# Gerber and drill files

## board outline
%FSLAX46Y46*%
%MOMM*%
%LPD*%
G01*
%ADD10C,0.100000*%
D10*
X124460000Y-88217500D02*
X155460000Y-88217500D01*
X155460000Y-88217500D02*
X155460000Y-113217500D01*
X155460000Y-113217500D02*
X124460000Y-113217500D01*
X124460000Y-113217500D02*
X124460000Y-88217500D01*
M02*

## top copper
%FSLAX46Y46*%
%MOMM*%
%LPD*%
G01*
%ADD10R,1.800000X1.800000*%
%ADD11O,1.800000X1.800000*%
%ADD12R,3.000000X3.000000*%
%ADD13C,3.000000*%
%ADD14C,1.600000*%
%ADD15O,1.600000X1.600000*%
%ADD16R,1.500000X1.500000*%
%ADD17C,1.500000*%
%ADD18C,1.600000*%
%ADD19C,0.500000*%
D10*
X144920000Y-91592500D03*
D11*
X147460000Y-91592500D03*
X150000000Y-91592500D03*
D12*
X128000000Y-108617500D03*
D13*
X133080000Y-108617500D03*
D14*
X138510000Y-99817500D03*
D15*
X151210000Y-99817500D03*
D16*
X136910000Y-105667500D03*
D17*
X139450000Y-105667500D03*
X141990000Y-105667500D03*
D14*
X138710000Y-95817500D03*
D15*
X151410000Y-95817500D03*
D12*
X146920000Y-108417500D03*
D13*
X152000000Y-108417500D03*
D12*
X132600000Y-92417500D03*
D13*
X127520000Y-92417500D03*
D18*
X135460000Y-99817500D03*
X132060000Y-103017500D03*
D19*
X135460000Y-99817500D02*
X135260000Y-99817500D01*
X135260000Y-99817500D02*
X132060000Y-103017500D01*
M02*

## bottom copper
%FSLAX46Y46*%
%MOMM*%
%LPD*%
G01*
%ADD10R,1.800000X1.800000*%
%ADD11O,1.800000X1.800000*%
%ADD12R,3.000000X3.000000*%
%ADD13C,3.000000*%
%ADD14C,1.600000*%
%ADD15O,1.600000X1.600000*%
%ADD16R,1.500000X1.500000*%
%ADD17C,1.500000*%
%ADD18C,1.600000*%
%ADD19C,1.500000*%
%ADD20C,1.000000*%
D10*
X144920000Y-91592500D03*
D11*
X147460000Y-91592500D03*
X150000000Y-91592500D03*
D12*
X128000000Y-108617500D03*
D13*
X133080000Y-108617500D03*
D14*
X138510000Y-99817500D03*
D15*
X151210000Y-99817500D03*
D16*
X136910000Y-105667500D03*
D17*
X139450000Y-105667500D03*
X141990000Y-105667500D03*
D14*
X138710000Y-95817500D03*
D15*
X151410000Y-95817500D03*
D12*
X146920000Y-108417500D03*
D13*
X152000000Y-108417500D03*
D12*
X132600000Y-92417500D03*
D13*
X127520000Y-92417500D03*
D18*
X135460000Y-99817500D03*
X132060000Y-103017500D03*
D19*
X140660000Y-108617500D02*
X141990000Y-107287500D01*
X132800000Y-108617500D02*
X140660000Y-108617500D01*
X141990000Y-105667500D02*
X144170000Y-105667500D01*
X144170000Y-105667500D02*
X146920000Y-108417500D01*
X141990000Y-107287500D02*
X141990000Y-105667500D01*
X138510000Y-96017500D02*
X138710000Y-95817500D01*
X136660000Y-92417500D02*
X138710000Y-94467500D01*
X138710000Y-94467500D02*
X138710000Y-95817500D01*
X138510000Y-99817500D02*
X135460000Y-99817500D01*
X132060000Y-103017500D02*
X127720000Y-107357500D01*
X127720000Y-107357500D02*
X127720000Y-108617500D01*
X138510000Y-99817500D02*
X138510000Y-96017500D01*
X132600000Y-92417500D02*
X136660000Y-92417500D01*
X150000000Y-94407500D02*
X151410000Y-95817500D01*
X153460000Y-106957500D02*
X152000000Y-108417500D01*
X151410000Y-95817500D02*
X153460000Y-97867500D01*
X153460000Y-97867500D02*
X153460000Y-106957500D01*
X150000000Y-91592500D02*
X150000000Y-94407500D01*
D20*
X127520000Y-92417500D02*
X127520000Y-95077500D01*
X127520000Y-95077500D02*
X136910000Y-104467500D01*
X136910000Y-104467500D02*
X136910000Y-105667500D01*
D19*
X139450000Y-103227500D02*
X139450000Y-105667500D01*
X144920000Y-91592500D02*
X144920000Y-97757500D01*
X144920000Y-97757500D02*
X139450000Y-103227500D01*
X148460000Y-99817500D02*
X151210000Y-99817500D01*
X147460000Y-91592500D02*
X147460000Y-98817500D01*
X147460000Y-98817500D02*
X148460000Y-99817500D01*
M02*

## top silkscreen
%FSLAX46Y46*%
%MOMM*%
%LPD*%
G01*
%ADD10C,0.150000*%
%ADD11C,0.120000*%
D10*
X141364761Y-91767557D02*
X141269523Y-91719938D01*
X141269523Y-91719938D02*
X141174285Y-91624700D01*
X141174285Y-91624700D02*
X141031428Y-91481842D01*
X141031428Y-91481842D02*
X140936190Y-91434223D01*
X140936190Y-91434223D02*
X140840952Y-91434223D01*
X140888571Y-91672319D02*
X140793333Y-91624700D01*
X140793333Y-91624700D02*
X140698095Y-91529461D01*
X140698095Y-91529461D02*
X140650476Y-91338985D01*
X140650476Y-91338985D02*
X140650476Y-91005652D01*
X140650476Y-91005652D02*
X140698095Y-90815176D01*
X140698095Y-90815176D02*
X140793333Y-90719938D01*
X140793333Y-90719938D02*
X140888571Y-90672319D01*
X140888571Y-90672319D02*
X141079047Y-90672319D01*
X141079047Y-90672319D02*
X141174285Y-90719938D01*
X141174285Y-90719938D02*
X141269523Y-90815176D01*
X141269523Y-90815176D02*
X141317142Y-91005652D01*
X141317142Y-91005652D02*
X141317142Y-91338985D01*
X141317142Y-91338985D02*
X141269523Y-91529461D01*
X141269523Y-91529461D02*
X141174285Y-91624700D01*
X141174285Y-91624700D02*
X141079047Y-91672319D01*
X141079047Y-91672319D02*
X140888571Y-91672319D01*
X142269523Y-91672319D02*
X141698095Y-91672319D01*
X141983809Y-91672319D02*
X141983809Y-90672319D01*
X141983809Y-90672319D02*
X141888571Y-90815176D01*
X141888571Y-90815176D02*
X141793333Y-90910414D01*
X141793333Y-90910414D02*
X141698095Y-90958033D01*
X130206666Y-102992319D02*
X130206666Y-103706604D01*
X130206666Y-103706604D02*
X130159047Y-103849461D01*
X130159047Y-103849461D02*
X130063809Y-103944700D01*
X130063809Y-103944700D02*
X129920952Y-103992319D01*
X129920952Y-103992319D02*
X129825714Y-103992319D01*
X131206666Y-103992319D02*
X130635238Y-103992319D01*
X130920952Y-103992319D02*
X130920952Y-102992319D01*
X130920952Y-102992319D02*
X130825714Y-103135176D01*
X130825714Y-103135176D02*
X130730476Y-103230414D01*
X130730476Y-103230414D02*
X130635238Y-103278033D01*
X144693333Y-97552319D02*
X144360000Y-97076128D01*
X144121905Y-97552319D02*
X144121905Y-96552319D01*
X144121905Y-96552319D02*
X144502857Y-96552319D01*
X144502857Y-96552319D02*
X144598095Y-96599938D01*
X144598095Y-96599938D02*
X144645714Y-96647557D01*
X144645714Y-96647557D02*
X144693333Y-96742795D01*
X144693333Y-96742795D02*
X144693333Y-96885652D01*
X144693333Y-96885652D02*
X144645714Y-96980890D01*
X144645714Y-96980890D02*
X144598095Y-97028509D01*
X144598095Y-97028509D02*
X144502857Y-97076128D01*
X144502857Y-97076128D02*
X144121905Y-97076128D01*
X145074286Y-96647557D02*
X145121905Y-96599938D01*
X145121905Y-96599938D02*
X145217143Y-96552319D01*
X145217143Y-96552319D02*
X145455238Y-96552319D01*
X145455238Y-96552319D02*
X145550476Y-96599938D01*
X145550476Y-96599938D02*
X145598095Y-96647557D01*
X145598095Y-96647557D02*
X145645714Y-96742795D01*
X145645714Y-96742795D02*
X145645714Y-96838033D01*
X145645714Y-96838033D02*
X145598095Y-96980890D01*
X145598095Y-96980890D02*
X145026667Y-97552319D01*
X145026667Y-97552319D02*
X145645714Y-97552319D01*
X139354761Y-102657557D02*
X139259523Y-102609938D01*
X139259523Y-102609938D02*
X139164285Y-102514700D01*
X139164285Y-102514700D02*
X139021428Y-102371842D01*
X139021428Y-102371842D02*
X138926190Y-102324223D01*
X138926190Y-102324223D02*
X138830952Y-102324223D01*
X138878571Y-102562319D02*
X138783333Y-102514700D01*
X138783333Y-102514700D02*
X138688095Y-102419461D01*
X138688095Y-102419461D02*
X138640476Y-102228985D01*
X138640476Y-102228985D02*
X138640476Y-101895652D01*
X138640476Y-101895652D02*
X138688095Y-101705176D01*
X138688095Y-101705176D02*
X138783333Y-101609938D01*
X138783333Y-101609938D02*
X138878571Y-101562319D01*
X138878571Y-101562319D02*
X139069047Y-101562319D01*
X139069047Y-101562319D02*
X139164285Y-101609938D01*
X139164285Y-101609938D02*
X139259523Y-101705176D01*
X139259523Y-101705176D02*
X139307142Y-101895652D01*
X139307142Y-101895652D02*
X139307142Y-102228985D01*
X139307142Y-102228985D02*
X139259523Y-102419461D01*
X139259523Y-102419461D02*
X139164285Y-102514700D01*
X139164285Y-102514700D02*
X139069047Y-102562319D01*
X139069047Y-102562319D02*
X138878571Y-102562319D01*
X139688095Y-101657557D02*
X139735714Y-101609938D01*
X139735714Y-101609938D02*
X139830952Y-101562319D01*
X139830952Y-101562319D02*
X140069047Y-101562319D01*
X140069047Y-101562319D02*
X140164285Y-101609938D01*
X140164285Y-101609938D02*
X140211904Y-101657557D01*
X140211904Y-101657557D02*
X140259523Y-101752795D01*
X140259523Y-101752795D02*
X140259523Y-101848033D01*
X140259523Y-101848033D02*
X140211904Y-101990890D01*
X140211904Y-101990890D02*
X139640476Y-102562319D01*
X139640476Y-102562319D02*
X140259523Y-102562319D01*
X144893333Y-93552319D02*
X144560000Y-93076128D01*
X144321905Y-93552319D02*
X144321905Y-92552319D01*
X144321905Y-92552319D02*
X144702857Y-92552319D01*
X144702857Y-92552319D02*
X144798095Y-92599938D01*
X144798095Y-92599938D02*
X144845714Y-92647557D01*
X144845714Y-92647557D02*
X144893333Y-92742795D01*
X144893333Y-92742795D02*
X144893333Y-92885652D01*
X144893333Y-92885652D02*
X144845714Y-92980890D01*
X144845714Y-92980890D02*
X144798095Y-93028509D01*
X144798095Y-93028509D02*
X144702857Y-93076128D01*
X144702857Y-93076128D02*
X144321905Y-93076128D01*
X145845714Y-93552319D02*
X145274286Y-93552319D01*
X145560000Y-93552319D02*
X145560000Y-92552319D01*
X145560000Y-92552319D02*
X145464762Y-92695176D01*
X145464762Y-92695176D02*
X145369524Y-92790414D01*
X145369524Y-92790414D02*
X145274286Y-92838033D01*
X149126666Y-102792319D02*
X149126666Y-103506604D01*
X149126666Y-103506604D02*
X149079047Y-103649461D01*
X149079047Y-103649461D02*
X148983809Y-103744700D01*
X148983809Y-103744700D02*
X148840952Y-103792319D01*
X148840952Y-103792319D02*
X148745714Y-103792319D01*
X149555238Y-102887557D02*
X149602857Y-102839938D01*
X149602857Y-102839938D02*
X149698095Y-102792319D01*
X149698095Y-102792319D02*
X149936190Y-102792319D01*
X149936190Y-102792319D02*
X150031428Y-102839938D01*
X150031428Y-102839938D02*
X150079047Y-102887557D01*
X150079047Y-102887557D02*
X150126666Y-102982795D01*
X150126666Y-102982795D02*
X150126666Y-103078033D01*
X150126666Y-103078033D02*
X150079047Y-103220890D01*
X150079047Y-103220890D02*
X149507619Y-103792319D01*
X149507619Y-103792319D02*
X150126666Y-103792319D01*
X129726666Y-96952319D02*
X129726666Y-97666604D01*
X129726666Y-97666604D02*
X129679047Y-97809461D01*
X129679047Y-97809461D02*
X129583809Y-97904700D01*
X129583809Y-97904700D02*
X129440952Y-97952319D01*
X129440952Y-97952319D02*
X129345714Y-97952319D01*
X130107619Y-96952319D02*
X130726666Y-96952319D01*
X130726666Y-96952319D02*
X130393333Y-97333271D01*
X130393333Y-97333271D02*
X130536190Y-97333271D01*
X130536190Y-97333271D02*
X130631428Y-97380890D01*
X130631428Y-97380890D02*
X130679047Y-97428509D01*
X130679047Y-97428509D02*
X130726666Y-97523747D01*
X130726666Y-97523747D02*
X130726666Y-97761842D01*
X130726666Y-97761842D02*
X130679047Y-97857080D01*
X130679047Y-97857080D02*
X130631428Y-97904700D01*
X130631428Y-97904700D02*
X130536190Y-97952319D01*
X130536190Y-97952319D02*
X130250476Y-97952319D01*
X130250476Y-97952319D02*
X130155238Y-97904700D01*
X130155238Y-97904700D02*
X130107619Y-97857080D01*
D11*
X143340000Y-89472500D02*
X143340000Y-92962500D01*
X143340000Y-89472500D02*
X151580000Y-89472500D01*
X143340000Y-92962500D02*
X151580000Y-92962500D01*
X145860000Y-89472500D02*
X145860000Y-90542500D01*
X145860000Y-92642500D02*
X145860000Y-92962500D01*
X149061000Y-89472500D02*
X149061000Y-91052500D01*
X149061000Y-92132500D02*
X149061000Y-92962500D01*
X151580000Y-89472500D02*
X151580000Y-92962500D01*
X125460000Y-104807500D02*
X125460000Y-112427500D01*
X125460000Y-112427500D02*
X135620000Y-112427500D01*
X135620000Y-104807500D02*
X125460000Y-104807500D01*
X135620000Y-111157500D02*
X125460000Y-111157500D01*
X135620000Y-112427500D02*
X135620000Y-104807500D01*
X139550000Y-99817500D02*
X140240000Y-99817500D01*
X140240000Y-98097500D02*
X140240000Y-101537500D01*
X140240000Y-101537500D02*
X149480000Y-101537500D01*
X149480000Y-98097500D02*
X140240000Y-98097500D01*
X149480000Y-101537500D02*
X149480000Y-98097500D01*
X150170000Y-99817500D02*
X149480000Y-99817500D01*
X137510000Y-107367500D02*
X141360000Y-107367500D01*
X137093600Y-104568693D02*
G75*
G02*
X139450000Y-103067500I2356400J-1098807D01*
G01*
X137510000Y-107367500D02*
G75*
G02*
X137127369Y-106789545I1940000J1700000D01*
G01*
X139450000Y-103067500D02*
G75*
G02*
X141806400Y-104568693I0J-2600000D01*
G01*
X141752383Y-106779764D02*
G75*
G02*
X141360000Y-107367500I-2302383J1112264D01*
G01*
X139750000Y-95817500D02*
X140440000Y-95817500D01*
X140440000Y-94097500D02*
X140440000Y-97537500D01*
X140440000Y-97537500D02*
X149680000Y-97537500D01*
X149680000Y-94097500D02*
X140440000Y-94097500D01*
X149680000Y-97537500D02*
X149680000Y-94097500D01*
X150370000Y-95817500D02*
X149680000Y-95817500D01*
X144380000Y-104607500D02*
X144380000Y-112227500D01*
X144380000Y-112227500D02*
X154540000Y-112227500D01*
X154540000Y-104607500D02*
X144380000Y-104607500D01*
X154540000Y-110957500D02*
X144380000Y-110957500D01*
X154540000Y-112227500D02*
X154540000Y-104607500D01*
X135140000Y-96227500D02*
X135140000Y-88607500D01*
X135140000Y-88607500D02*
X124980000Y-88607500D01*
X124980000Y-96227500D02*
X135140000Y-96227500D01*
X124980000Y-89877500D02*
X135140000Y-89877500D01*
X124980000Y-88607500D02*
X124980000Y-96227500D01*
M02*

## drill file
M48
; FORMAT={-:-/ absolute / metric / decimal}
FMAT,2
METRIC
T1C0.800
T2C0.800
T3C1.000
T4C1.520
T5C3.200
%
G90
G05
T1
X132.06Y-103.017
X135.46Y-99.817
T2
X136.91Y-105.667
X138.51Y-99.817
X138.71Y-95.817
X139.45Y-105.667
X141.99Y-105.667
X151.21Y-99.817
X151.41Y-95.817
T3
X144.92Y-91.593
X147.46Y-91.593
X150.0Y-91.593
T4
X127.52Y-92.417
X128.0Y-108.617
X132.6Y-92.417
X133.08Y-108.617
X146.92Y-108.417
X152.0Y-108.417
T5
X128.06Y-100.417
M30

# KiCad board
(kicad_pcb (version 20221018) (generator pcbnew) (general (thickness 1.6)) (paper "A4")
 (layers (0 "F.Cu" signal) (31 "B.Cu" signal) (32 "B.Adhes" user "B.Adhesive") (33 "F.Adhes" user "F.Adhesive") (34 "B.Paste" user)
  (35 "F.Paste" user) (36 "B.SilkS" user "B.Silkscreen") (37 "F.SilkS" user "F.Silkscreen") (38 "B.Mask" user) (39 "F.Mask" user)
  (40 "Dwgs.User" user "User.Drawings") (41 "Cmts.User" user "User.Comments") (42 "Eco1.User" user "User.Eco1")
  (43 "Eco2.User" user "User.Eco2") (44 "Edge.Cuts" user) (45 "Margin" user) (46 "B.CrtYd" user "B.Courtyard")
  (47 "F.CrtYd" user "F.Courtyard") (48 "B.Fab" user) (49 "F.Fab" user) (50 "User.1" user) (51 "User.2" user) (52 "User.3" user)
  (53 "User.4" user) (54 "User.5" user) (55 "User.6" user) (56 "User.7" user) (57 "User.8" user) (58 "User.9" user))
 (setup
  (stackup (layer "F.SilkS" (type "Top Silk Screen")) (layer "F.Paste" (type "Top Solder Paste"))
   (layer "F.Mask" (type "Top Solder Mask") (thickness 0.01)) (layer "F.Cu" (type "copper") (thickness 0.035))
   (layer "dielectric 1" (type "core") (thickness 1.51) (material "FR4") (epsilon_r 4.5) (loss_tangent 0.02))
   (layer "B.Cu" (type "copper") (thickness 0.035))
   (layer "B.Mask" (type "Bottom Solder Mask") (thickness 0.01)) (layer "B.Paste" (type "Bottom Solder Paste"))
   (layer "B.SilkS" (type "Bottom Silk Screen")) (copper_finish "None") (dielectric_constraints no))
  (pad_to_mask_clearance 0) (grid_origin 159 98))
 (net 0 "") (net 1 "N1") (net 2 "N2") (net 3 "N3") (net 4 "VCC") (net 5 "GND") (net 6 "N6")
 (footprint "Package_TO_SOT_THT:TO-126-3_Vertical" (layer "F.Cu") (at 144.92 91.5925)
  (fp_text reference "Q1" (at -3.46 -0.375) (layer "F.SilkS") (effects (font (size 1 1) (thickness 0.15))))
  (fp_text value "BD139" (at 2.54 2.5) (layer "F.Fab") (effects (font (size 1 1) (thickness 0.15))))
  (fp_line (start -1.58 -2.12) (end -1.58 1.37) (stroke (width 0.12) (type solid)) (layer "F.SilkS"))
  (fp_line (start -1.58 -2.12) (end 6.66 -2.12) (stroke (width 0.12) (type solid)) (layer "F.SilkS"))
  (fp_line (start -1.58 1.37) (end 6.66 1.37) (stroke (width 0.12) (type solid)) (layer "F.SilkS"))
  (fp_line (start 0.94 -2.12) (end 0.94 -1.05) (stroke (width 0.12) (type solid)) (layer "F.SilkS"))
  (fp_line (start 0.94 1.05) (end 0.94 1.37) (stroke (width 0.12) (type solid)) (layer "F.SilkS"))
  (fp_line (start 4.141 -2.12) (end 4.141 -0.54) (stroke (width 0.12) (type solid)) (layer "F.SilkS"))
  (fp_line (start 4.141 0.54) (end 4.141 1.37) (stroke (width 0.12) (type solid)) (layer "F.SilkS"))
  (fp_line (start 6.66 -2.12) (end 6.66 1.37) (stroke (width 0.12) (type solid)) (layer "F.SilkS"))
  (pad "1" thru_hole rect (at 0 0) (size 1.8 1.8) (drill 1) (layers "*.Cu" "*.Mask") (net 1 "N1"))
  (pad "2" thru_hole oval (at 2.54 0) (size 1.8 1.8) (drill 1) (layers "*.Cu" "*.Mask") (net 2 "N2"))
  (pad "3" thru_hole oval (at 5.08 0) (size 1.8 1.8) (drill 1) (layers "*.Cu" "*.Mask") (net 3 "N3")))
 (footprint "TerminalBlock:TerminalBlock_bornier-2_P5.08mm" (layer "F.Cu") (at 128 108.6175)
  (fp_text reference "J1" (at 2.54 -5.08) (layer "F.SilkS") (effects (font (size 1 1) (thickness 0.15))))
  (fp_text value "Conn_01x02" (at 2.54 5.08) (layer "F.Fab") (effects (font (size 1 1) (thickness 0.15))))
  (fp_line (start -2.54 -3.81) (end -2.54 3.81) (stroke (width 0.12) (type solid)) (layer "F.SilkS"))
  (fp_line (start -2.54 3.81) (end 7.62 3.81) (stroke (width 0.12) (type solid)) (layer "F.SilkS"))
  (fp_line (start 7.62 -3.81) (end -2.54 -3.81) (stroke (width 0.12) (type solid)) (layer "F.SilkS"))
  (fp_line (start 7.62 2.54) (end -2.54 2.54) (stroke (width 0.12) (type solid)) (layer "F.SilkS"))
  (fp_line (start 7.62 3.81) (end 7.62 -3.81) (stroke (width 0.12) (type solid)) (layer "F.SilkS"))
  (pad "1" thru_hole rect (at 0 0) (size 3 3) (drill 1.52) (layers "*.Cu" "*.Mask") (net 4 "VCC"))
  (pad "2" thru_hole circle (at 5.08 0) (size 3 3) (drill 1.52) (layers "*.Cu" "*.Mask") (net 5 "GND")))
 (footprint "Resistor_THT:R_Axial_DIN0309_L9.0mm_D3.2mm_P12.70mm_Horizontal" (layer "F.Cu") (at 138.51 99.8175)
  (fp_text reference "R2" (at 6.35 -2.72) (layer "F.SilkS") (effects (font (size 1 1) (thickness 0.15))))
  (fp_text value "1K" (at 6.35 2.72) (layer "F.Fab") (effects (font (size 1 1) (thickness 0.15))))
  (fp_line (start 1.04 0) (end 1.73 0) (stroke (width 0.12) (type solid)) (layer "F.SilkS"))
  (fp_line (start 1.73 -1.72) (end 1.73 1.72) (stroke (width 0.12) (type solid)) (layer "F.SilkS"))
  (fp_line (start 1.73 1.72) (end 10.97 1.72) (stroke (width 0.12) (type solid)) (layer "F.SilkS"))
  (fp_line (start 10.97 -1.72) (end 1.73 -1.72) (stroke (width 0.12) (type solid)) (layer "F.SilkS"))
  (fp_line (start 10.97 1.72) (end 10.97 -1.72) (stroke (width 0.12) (type solid)) (layer "F.SilkS"))
  (fp_line (start 11.66 0) (end 10.97 0) (stroke (width 0.12) (type solid)) (layer "F.SilkS"))
  (pad "1" thru_hole circle (at 0 0) (size 1.6 1.6) (drill 0.8) (layers "*.Cu" "*.Mask") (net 4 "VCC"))
  (pad "2" thru_hole oval (at 12.7 0) (size 1.6 1.6) (drill 0.8) (layers "*.Cu" "*.Mask") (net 2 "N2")))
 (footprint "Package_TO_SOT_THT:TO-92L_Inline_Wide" (layer "F.Cu") (at 136.91 105.6675)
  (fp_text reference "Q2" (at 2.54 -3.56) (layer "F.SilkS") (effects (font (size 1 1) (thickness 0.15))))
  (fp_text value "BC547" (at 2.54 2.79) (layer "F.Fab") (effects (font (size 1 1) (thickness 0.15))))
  (fp_line (start 0.6 1.7) (end 4.45 1.7) (stroke (width 0.12) (type solid)) (layer "F.SilkS"))
  (fp_arc (start 0.1836 -1.098807) (mid 1.143021 -2.192817) (end 2.54 -2.6) (stroke (width 0.12) (type solid)) (layer "F.SilkS"))
  (fp_arc (start 0.6 1.7) (mid 0.389183 1.423933) (end 0.217369 1.122045) (stroke (width 0.12) (type solid)) (layer "F.SilkS"))
  (fp_arc (start 2.54 -2.6) (mid 3.936979 -2.192818) (end 4.8964 -1.098807) (stroke (width 0.12) (type solid)) (layer "F.SilkS"))
  (fp_arc (start 4.842383 1.112264) (mid 4.666594 1.419753) (end 4.45 1.7) (stroke (width 0.12) (type solid)) (layer "F.SilkS"))
  (pad "1" thru_hole rect (at 0 0) (size 1.5 1.5) (drill 0.8) (layers "*.Cu" "*.Mask") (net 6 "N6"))
  (pad "2" thru_hole circle (at 2.54 0) (size 1.5 1.5) (drill 0.8) (layers "*.Cu" "*.Mask") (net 1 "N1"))
  (pad "3" thru_hole circle (at 5.08 0) (size 1.5 1.5) (drill 0.8) (layers "*.Cu" "*.Mask") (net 5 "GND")))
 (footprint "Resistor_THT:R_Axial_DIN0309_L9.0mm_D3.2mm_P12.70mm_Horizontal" (layer "F.Cu") (at 138.71 95.8175)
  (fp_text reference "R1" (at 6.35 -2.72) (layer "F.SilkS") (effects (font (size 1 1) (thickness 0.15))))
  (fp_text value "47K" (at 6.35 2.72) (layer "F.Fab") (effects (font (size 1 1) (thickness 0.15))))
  (fp_line (start 1.04 0) (end 1.73 0) (stroke (width 0.12) (type solid)) (layer "F.SilkS"))
  (fp_line (start 1.73 -1.72) (end 1.73 1.72) (stroke (width 0.12) (type solid)) (layer "F.SilkS"))
  (fp_line (start 1.73 1.72) (end 10.97 1.72) (stroke (width 0.12) (type solid)) (layer "F.SilkS"))
  (fp_line (start 10.97 -1.72) (end 1.73 -1.72) (stroke (width 0.12) (type solid)) (layer "F.SilkS"))
  (fp_line (start 10.97 1.72) (end 10.97 -1.72) (stroke (width 0.12) (type solid)) (layer "F.SilkS"))
  (fp_line (start 11.66 0) (end 10.97 0) (stroke (width 0.12) (type solid)) (layer "F.SilkS"))
  (pad "1" thru_hole circle (at 0 0) (size 1.6 1.6) (drill 0.8) (layers "*.Cu" "*.Mask") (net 4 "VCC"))
  (pad "2" thru_hole oval (at 12.7 0) (size 1.6 1.6) (drill 0.8) (layers "*.Cu" "*.Mask") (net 3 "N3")))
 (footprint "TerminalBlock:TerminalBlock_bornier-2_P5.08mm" (layer "F.Cu") (at 146.92 108.4175)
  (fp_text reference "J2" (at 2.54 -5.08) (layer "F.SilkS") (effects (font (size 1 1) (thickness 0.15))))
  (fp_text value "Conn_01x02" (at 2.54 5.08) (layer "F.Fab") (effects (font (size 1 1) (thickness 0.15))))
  (fp_line (start -2.54 -3.81) (end -2.54 3.81) (stroke (width 0.12) (type solid)) (layer "F.SilkS"))
  (fp_line (start -2.54 3.81) (end 7.62 3.81) (stroke (width 0.12) (type solid)) (layer "F.SilkS"))
  (fp_line (start 7.62 -3.81) (end -2.54 -3.81) (stroke (width 0.12) (type solid)) (layer "F.SilkS"))
  (fp_line (start 7.62 2.54) (end -2.54 2.54) (stroke (width 0.12) (type solid)) (layer "F.SilkS"))
  (fp_line (start 7.62 3.81) (end 7.62 -3.81) (stroke (width 0.12) (type solid)) (layer "F.SilkS"))
  (pad "1" thru_hole rect (at 0 0) (size 3 3) (drill 1.52) (layers "*.Cu" "*.Mask") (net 5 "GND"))
  (pad "2" thru_hole circle (at 5.08 0) (size 3 3) (drill 1.52) (layers "*.Cu" "*.Mask") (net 3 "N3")))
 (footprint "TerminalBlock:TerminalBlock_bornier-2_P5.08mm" (layer "F.Cu") (at 132.6 92.4175 180)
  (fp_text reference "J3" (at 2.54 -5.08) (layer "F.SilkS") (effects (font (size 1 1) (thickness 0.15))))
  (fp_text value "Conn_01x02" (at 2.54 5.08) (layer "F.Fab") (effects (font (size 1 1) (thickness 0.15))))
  (fp_line (start -2.54 -3.81) (end -2.54 3.81) (stroke (width 0.12) (type solid)) (layer "F.SilkS"))
  (fp_line (start -2.54 3.81) (end 7.62 3.81) (stroke (width 0.12) (type solid)) (layer "F.SilkS"))
  (fp_line (start 7.62 -3.81) (end -2.54 -3.81) (stroke (width 0.12) (type solid)) (layer "F.SilkS"))
  (fp_line (start 7.62 2.54) (end -2.54 2.54) (stroke (width 0.12) (type solid)) (layer "F.SilkS"))
  (fp_line (start 7.62 3.81) (end 7.62 -3.81) (stroke (width 0.12) (type solid)) (layer "F.SilkS"))
  (pad "1" thru_hole rect (at 0 0 180) (size 3 3) (drill 1.52) (layers "*.Cu" "*.Mask") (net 4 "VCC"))
  (pad "2" thru_hole circle (at 5.08 0 180) (size 3 3) (drill 1.52) (layers "*.Cu" "*.Mask") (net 6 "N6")))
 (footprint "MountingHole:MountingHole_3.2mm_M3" (layer "F.Cu") (at 128.06 100.4175)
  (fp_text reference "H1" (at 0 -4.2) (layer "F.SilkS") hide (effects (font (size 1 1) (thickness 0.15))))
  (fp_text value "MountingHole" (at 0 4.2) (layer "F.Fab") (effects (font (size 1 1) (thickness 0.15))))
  (pad "" np_thru_hole circle (at 0 0) (size 3.2 3.2) (drill 3.2) (layers "*.Cu" "*.Mask")))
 (gr_line (start 124.46 88.2175) (end 155.46 88.2175) (stroke (width 0.1) (type solid)) (layer "Edge.Cuts"))
 (gr_line (start 155.46 88.2175) (end 155.46 113.2175) (stroke (width 0.1) (type solid)) (layer "Edge.Cuts"))
 (gr_line (start 155.46 113.2175) (end 124.46 113.2175) (stroke (width 0.1) (type solid)) (layer "Edge.Cuts"))
 (gr_line (start 124.46 113.2175) (end 124.46 88.2175) (stroke (width 0.1) (type solid)) (layer "Edge.Cuts"))
 (segment (start 140.66 108.6175) (end 141.99 107.2875) (width 1.5) (layer "B.Cu") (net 5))
 (segment (start 132.8 108.6175) (end 140.66 108.6175) (width 1.5) (layer "B.Cu") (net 5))
 (segment (start 141.99 105.6675) (end 144.17 105.6675) (width 1.5) (layer "B.Cu") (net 5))
 (segment (start 144.17 105.6675) (end 146.92 108.4175) (width 1.5) (layer "B.Cu") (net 5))
 (segment (start 141.99 107.2875) (end 141.99 105.6675) (width 1.5) (layer "B.Cu") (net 5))
 (segment (start 135.46 99.8175) (end 135.26 99.8175) (width 0.5) (layer "F.Cu") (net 4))
 (segment (start 135.26 99.8175) (end 132.06 103.0175) (width 0.5) (layer "F.Cu") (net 4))
 (via (at 135.46 99.8175) (size 1.6) (drill 0.8) (layers "F.Cu" "B.Cu") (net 4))
 (via (at 132.06 103.0175) (size 1.6) (drill 0.8) (layers "F.Cu" "B.Cu") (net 4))
 (segment (start 138.51 96.0175) (end 138.71 95.8175) (width 1.5) (layer "B.Cu") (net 4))
 (segment (start 136.66 92.4175) (end 138.71 94.4675) (width 1.5) (layer "B.Cu") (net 4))
 (segment (start 138.71 94.4675) (end 138.71 95.8175) (width 1.5) (layer "B.Cu") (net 4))
 (segment (start 138.51 99.8175) (end 135.46 99.8175) (width 1.5) (layer "B.Cu") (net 4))
 (segment (start 132.06 103.0175) (end 127.72 107.3575) (width 1.5) (layer "B.Cu") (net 4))
 (segment (start 127.72 107.3575) (end 127.72 108.6175) (width 1.5) (layer "B.Cu") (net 4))
 (segment (start 138.51 99.8175) (end 138.51 96.0175) (width 1.5) (layer "B.Cu") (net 4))
 (segment (start 132.6 92.4175) (end 136.66 92.4175) (width 1.5) (layer "B.Cu") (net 4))
 (segment (start 150 94.4075) (end 151.41 95.8175) (width 1.5) (layer "B.Cu") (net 3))
 (segment (start 153.46 106.9575) (end 152 108.4175) (width 1.5) (layer "B.Cu") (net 3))
 (segment (start 151.41 95.8175) (end 153.46 97.8675) (width 1.5) (layer "B.Cu") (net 3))
 (segment (start 153.46 97.8675) (end 153.46 106.9575) (width 1.5) (layer "B.Cu") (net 3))
 (segment (start 150 91.5925) (end 150 94.4075) (width 1.5) (layer "B.Cu") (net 3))
 (segment (start 127.52 92.4175) (end 127.52 95.0775) (width 1) (layer "B.Cu") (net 6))
 (segment (start 127.52 95.0775) (end 136.91 104.4675) (width 1) (layer "B.Cu") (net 6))
 (segment (start 136.91 104.4675) (end 136.91 105.6675) (width 1) (layer "B.Cu") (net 6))
 (segment (start 139.45 103.2275) (end 139.45 105.6675) (width 1.5) (layer "B.Cu") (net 1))
 (segment (start 144.92 91.5925) (end 144.92 97.7575) (width 1.5) (layer "B.Cu") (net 1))
 (segment (start 144.92 97.7575) (end 139.45 103.2275) (width 1.5) (layer "B.Cu") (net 1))
 (segment (start 148.46 99.8175) (end 151.21 99.8175) (width 1.5) (layer "B.Cu") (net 2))
 (segment (start 147.46 91.5925) (end 147.46 98.8175) (width 1.5) (layer "B.Cu") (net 2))
 (segment (start 147.46 98.8175) (end 148.46 99.8175) (width 1.5) (layer "B.Cu") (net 2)))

